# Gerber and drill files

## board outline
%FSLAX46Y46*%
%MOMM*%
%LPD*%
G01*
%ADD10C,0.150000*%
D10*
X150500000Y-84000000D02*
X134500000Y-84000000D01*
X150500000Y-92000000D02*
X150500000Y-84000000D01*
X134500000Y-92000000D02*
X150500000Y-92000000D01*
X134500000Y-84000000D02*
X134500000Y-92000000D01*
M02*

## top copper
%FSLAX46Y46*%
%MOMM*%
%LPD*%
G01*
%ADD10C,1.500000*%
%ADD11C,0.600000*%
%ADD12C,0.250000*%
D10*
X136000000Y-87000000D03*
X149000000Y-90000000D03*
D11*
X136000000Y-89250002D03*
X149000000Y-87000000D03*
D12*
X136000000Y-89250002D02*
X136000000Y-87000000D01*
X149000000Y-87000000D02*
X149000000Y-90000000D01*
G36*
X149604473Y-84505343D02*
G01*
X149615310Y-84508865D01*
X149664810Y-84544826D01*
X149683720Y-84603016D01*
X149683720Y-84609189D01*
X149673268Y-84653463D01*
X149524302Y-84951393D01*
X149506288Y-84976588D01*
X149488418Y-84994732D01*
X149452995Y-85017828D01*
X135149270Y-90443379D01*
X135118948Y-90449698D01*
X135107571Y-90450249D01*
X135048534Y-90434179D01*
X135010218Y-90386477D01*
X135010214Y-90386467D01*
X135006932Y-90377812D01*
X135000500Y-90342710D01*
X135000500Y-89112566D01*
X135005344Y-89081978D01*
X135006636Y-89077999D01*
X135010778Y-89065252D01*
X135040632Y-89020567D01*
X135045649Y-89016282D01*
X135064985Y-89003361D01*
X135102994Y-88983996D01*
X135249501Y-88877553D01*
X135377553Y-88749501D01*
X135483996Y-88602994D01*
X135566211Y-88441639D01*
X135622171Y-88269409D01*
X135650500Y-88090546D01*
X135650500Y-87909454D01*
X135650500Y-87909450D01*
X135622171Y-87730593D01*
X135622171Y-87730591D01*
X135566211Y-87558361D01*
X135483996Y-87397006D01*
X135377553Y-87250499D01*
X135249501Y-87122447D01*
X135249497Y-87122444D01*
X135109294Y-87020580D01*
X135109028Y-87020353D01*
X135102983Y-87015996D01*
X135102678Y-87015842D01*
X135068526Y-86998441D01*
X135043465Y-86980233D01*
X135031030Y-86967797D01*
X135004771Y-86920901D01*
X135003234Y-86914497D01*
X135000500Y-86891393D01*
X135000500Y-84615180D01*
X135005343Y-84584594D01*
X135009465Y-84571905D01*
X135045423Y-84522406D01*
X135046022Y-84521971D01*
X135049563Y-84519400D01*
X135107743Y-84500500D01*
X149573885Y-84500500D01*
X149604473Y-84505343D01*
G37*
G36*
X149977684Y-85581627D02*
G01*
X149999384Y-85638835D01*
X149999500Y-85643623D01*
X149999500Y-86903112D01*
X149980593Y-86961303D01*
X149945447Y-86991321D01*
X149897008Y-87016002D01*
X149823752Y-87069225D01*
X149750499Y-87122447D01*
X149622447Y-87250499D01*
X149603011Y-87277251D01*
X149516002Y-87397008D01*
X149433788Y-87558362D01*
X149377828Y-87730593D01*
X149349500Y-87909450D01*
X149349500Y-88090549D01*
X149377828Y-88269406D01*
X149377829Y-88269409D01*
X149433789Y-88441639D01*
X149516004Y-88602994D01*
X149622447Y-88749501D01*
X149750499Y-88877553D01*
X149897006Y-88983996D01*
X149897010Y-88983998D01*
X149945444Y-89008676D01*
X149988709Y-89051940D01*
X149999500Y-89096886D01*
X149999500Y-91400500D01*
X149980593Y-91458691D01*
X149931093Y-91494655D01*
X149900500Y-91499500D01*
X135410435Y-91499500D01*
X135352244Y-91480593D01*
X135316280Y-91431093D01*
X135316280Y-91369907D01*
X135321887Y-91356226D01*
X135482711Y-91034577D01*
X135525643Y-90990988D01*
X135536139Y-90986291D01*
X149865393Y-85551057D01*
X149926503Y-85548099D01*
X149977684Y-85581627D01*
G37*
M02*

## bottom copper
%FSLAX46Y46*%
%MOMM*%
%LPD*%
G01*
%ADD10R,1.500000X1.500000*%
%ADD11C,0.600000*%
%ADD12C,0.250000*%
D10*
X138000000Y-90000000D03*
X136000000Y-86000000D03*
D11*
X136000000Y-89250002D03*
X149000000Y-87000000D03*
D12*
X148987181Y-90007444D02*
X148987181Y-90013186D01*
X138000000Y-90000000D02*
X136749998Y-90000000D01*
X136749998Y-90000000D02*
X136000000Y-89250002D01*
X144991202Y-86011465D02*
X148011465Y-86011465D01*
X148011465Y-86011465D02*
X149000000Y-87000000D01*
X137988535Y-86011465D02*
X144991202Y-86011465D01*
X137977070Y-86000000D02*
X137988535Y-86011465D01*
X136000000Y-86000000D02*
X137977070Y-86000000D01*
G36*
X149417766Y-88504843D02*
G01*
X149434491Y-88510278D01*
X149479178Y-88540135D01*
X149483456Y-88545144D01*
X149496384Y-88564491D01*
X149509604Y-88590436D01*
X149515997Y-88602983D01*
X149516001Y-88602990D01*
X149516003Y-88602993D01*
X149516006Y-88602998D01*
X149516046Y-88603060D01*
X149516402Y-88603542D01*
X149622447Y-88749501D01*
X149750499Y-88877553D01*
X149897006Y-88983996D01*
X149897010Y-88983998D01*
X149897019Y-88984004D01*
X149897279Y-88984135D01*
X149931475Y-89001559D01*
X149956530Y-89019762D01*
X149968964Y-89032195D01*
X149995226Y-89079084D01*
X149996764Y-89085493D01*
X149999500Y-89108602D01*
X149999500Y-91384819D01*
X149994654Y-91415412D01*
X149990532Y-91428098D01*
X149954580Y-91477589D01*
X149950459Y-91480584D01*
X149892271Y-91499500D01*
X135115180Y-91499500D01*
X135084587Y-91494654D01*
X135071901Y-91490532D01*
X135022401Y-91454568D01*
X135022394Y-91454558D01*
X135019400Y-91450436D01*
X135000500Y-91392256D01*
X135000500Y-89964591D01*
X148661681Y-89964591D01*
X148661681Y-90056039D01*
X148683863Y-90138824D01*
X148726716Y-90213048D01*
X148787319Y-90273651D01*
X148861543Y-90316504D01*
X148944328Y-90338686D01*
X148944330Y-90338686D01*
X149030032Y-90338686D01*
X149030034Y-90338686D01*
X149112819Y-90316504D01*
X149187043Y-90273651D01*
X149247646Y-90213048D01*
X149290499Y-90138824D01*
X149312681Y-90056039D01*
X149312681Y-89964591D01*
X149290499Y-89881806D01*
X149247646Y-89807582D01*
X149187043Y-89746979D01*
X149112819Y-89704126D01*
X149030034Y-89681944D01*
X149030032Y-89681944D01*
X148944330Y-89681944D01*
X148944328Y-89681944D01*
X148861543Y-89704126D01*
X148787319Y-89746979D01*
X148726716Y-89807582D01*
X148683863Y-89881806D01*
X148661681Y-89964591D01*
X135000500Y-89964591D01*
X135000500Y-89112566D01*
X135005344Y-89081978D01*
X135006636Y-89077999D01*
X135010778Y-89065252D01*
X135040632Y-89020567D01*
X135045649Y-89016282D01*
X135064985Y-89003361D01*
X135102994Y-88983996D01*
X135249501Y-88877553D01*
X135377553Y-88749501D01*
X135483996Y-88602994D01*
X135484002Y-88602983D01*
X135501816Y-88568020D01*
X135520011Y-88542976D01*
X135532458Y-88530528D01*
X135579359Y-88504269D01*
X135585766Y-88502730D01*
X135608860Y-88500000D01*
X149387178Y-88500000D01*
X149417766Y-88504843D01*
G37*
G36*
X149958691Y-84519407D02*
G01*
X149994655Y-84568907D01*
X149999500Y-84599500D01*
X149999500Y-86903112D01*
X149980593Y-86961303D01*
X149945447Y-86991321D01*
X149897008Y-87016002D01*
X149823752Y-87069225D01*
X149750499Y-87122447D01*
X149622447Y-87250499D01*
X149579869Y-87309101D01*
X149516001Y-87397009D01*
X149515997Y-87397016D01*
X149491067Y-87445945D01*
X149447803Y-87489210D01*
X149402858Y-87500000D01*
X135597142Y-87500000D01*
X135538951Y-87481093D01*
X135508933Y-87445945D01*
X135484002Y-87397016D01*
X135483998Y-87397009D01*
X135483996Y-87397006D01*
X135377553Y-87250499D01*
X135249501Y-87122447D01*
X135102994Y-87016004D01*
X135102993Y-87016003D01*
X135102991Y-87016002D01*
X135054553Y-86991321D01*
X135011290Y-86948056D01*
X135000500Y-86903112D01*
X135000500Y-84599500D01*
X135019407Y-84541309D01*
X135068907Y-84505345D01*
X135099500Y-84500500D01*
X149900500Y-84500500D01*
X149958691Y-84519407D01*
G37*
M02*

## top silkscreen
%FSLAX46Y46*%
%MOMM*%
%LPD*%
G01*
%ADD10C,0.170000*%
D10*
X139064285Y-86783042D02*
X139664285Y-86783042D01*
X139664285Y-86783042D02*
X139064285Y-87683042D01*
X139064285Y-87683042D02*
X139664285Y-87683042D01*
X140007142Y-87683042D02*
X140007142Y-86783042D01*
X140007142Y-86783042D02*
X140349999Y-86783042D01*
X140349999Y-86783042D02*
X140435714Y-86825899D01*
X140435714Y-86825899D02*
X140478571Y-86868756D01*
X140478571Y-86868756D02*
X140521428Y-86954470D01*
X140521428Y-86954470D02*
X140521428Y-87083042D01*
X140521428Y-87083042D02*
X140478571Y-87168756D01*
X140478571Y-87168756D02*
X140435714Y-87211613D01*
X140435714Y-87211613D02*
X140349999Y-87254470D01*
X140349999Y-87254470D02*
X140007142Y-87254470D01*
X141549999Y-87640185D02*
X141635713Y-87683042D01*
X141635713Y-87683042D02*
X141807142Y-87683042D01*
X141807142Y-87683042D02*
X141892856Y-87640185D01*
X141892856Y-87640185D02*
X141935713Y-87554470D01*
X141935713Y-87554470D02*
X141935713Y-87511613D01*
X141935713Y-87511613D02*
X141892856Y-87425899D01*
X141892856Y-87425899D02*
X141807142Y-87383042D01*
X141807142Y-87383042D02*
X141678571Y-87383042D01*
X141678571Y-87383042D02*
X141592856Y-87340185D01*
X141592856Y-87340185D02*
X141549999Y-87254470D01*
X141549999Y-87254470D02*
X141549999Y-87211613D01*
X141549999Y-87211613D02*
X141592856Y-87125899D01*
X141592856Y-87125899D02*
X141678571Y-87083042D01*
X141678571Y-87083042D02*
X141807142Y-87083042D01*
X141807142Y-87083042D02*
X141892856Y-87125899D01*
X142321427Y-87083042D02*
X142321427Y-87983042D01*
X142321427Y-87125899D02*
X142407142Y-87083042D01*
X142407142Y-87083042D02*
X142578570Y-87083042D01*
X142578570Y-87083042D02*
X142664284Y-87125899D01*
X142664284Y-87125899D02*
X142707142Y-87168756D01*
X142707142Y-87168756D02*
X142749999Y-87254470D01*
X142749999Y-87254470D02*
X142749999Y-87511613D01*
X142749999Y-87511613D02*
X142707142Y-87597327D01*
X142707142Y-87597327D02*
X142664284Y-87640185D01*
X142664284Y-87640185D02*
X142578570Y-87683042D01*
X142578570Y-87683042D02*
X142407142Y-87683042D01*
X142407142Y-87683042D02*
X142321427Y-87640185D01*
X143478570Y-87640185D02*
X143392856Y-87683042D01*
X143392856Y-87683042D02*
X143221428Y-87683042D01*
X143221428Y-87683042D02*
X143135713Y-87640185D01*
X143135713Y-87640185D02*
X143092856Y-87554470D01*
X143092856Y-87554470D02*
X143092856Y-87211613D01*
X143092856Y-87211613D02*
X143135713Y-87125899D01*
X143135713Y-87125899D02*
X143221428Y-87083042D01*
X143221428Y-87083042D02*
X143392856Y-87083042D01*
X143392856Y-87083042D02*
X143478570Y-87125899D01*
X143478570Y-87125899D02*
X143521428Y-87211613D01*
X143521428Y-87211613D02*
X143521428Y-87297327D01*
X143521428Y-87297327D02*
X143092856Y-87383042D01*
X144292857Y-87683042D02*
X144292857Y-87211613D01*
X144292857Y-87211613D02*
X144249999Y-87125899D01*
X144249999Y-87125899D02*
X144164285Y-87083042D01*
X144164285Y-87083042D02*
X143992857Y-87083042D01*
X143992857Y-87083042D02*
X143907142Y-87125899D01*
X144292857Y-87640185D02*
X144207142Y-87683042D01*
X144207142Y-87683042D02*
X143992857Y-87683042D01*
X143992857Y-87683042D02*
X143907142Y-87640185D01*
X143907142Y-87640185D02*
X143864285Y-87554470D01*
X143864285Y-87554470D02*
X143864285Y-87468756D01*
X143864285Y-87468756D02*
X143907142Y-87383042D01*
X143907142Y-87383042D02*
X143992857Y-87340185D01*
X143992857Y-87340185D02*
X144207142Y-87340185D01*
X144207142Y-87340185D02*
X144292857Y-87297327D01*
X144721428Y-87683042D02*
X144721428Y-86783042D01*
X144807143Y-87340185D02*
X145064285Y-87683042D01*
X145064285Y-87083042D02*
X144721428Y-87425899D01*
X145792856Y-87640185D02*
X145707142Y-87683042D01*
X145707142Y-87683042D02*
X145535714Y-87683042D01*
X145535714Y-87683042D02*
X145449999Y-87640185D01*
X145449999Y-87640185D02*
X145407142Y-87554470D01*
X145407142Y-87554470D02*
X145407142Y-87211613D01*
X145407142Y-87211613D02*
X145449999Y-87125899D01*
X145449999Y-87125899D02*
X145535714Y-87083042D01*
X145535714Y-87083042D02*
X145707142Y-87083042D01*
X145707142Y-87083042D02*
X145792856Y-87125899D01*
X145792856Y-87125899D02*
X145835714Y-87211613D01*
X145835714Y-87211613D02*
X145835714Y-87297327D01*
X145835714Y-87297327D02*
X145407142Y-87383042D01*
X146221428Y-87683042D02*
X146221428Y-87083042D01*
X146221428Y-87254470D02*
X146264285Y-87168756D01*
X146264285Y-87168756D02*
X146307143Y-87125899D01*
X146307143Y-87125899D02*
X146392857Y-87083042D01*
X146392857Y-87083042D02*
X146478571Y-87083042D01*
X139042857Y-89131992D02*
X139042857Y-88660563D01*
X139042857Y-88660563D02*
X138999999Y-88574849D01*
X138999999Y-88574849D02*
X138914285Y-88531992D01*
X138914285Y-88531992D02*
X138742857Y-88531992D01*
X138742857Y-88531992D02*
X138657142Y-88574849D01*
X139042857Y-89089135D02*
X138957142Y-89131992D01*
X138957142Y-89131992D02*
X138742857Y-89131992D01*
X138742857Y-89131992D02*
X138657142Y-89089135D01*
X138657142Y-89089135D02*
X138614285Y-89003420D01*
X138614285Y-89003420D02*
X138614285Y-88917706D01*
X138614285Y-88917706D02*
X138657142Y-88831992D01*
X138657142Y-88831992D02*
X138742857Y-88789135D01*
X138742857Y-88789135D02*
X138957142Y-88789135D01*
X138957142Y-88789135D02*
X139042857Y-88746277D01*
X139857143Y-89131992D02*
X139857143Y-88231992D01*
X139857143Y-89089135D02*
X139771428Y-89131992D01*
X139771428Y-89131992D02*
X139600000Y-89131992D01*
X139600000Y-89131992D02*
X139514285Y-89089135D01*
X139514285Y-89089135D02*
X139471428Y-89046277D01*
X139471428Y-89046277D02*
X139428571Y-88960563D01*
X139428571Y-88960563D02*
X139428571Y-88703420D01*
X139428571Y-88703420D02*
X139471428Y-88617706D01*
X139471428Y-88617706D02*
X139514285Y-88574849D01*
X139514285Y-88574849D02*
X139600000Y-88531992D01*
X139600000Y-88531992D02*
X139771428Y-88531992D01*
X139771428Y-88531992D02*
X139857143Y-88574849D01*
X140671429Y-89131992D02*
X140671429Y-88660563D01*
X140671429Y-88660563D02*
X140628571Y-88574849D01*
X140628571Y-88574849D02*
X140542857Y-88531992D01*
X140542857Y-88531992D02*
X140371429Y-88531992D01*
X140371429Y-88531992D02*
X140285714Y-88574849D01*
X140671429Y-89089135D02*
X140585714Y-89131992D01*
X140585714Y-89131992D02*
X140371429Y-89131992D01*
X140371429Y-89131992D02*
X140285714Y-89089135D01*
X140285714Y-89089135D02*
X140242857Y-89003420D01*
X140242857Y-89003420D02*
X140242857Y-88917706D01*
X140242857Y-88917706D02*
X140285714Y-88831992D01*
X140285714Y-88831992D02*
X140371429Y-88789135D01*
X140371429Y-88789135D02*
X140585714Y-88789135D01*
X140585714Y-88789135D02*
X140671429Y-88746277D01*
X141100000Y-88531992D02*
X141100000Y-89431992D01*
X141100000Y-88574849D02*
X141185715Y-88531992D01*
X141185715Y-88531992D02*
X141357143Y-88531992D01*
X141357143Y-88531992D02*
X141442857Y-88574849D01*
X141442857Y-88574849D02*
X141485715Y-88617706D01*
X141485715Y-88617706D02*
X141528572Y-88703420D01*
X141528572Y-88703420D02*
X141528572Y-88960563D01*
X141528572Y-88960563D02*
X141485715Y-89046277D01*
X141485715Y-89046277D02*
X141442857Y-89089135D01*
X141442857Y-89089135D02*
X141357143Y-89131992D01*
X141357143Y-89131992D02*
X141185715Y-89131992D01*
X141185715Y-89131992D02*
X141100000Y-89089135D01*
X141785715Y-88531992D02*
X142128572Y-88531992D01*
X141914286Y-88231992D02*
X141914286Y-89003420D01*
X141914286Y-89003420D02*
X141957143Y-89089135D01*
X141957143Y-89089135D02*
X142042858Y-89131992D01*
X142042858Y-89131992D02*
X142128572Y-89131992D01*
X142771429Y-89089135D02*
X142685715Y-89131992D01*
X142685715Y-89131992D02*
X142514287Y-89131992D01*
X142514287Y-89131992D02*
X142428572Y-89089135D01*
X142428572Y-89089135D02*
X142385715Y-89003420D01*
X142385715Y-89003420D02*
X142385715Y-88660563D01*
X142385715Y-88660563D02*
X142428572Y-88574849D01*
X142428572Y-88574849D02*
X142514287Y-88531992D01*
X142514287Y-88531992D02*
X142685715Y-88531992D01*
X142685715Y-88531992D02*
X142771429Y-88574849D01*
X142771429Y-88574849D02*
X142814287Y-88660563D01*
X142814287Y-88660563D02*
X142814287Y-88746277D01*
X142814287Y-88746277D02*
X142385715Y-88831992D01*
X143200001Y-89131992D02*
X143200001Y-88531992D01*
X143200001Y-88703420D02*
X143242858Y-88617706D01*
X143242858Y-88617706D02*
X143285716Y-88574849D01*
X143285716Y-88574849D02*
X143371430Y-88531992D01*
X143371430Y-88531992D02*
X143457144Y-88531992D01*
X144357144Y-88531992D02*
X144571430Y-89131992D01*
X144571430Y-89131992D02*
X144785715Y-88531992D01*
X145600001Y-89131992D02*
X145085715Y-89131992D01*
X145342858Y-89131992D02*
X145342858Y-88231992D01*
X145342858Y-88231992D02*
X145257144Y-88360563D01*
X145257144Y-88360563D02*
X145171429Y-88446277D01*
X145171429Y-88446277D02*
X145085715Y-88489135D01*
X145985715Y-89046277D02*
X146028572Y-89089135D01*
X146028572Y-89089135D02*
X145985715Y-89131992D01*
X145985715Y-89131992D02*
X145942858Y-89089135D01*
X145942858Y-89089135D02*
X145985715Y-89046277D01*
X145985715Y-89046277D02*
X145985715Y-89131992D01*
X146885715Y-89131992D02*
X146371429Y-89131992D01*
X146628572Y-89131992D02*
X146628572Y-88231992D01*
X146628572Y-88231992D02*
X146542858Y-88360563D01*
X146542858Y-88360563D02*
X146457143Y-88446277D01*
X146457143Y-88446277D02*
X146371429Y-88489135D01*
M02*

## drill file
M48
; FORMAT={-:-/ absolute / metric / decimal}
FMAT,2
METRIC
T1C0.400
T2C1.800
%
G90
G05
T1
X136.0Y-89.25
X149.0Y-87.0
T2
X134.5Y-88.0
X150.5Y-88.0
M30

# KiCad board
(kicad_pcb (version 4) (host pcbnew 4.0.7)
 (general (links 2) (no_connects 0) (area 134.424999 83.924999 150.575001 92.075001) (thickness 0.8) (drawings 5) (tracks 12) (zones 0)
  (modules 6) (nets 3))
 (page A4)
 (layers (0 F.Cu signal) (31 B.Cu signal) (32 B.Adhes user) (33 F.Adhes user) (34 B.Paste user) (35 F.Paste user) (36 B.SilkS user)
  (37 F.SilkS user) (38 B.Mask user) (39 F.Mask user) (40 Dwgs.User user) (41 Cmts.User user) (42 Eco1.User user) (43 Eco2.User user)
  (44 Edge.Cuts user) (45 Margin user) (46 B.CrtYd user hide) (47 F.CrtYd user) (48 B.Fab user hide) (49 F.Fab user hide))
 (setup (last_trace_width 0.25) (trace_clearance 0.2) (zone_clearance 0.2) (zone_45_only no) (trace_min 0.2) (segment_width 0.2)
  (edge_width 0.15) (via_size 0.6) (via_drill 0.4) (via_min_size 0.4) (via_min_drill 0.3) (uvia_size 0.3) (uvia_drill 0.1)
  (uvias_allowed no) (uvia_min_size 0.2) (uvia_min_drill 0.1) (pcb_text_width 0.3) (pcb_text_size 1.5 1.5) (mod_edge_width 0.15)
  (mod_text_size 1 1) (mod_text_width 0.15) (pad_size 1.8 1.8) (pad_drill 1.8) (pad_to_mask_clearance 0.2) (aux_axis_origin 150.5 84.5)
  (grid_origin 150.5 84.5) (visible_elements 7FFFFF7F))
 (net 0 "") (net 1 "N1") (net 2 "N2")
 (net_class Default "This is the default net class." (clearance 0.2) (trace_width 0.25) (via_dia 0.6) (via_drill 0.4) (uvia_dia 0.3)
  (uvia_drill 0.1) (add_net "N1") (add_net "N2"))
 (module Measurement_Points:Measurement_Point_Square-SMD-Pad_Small (layer B.Cu) (at 138 90)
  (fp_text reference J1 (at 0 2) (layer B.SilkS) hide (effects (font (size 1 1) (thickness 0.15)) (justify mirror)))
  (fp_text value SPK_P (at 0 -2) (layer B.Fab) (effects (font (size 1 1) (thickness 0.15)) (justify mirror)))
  (pad 1 smd rect (at 0 0) (size 1.5 1.5) (layers B.Cu) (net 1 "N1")))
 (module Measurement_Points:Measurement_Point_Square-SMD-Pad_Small (layer B.Cu) (at 136 86)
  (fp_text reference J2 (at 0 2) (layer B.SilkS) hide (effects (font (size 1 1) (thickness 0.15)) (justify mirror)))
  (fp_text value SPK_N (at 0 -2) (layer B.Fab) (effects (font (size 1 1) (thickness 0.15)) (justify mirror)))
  (pad 1 smd rect (at 0 0) (size 1.5 1.5) (layers B.Cu) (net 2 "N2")))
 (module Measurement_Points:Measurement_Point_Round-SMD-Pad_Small (layer F.Cu) (at 136 87)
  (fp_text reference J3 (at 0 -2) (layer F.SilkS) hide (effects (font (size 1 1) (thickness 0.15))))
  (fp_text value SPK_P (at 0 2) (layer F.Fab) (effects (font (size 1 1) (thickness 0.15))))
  (pad 1 smd circle (at 0 0) (size 1.5 1.5) (layers F.Cu) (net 1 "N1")))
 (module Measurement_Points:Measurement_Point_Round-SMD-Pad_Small (layer F.Cu) (at 149 90)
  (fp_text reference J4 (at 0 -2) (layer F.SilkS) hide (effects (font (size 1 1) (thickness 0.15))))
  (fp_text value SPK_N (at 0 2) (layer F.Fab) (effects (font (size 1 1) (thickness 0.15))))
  (pad 1 smd circle (at 0 0) (size 1.5 1.5) (layers F.Cu) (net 2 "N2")))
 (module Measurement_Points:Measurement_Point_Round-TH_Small (layer F.Cu) (at 134.5 88)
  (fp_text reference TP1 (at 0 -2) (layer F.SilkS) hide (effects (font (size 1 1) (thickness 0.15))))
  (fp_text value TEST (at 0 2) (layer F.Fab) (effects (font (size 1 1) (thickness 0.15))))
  (pad "" np_thru_hole circle (at 0 0) (size 1.8 1.8) (drill 1.8) (layers *.Cu)))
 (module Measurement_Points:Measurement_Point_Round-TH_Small (layer F.Cu) (at 150.5 88)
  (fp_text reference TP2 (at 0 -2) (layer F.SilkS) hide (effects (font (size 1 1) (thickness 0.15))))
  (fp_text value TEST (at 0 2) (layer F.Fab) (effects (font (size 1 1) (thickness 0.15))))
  (pad "" np_thru_hole circle (at 0 0) (size 1.8 1.8) (drill 1.8) (layers *.Cu)))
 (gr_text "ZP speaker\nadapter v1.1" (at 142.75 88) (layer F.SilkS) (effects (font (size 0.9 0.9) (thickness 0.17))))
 (gr_line (start 150.5 84) (end 134.5 84) (layer Edge.Cuts) (width 0.15))
 (gr_line (start 150.5 92) (end 150.5 84) (layer Edge.Cuts) (width 0.15))
 (gr_line (start 134.5 92) (end 150.5 92) (layer Edge.Cuts) (width 0.15))
 (gr_line (start 134.5 84) (end 134.5 92) (layer Edge.Cuts) (width 0.15))
 (segment (start 148.987181 90.007444) (end 148.987181 90.013186) (width 0.25) (layer B.Cu) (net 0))
 (segment (start 136 89.250002) (end 136 87) (width 0.25) (layer F.Cu) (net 1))
 (segment (start 138 90) (end 136.749998 90) (width 0.25) (layer B.Cu) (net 1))
 (segment (start 136.749998 90) (end 136 89.250002) (width 0.25) (layer B.Cu) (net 1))
 (via (at 136 89.250002) (size 0.6) (drill 0.4) (layers F.Cu B.Cu) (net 1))
 (segment (start 149 87) (end 149 90) (width 0.25) (layer F.Cu) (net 2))
 (segment (start 144.991202 86.011465) (end 148.011465 86.011465) (width 0.25) (layer B.Cu) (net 2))
 (segment (start 148.011465 86.011465) (end 149 87) (width 0.25) (layer B.Cu) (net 2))
 (via (at 149 87) (size 0.6) (drill 0.4) (layers F.Cu B.Cu) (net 2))
 (segment (start 137.988535 86.011465) (end 144.991202 86.011465) (width 0.25) (layer B.Cu) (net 2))
 (segment (start 137.97707 86) (end 137.988535 86.011465) (width 0.25) (layer B.Cu) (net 2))
 (segment (start 136 86) (end 137.97707 86) (width 0.25) (layer B.Cu) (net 2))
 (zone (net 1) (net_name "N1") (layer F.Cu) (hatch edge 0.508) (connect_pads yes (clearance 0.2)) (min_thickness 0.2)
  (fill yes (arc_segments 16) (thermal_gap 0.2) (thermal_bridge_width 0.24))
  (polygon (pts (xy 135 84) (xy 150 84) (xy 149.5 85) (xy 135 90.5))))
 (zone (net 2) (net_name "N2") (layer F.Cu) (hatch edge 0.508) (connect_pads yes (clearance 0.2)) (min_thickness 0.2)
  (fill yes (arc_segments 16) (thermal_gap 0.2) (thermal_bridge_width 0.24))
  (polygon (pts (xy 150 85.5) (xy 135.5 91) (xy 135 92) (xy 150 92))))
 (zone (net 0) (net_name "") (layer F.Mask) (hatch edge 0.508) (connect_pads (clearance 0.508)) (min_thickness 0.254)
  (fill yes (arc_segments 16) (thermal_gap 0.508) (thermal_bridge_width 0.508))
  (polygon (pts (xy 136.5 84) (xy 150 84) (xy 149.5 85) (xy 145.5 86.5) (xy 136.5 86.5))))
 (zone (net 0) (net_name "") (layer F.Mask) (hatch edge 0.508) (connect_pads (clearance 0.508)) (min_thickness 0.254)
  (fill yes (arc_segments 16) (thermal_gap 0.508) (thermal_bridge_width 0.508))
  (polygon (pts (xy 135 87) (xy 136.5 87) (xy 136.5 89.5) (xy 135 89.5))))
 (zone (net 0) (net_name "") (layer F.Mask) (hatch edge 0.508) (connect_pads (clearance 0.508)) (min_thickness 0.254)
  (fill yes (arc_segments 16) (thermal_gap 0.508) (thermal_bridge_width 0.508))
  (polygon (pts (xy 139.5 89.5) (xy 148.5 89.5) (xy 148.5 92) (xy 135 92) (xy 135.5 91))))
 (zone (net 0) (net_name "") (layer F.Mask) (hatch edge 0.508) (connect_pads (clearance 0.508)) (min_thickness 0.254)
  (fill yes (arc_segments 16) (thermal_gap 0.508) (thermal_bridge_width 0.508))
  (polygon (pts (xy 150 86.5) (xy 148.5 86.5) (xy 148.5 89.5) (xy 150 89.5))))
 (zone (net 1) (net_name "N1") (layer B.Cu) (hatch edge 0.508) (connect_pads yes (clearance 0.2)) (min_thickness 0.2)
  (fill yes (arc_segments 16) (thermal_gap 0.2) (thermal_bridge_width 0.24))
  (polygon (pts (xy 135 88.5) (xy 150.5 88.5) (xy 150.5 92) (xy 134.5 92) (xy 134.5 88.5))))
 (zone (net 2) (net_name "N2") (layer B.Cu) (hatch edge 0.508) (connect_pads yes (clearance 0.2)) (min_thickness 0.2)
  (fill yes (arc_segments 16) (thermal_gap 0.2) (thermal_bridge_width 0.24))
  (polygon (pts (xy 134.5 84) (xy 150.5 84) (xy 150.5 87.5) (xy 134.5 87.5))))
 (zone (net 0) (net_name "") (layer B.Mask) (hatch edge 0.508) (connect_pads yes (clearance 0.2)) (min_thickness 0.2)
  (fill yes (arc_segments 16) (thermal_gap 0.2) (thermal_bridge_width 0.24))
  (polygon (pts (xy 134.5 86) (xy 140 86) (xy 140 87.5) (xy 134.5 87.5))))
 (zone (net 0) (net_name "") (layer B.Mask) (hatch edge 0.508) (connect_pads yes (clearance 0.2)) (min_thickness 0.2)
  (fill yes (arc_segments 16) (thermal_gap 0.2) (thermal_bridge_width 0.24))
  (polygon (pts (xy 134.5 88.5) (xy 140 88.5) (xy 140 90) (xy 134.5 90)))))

